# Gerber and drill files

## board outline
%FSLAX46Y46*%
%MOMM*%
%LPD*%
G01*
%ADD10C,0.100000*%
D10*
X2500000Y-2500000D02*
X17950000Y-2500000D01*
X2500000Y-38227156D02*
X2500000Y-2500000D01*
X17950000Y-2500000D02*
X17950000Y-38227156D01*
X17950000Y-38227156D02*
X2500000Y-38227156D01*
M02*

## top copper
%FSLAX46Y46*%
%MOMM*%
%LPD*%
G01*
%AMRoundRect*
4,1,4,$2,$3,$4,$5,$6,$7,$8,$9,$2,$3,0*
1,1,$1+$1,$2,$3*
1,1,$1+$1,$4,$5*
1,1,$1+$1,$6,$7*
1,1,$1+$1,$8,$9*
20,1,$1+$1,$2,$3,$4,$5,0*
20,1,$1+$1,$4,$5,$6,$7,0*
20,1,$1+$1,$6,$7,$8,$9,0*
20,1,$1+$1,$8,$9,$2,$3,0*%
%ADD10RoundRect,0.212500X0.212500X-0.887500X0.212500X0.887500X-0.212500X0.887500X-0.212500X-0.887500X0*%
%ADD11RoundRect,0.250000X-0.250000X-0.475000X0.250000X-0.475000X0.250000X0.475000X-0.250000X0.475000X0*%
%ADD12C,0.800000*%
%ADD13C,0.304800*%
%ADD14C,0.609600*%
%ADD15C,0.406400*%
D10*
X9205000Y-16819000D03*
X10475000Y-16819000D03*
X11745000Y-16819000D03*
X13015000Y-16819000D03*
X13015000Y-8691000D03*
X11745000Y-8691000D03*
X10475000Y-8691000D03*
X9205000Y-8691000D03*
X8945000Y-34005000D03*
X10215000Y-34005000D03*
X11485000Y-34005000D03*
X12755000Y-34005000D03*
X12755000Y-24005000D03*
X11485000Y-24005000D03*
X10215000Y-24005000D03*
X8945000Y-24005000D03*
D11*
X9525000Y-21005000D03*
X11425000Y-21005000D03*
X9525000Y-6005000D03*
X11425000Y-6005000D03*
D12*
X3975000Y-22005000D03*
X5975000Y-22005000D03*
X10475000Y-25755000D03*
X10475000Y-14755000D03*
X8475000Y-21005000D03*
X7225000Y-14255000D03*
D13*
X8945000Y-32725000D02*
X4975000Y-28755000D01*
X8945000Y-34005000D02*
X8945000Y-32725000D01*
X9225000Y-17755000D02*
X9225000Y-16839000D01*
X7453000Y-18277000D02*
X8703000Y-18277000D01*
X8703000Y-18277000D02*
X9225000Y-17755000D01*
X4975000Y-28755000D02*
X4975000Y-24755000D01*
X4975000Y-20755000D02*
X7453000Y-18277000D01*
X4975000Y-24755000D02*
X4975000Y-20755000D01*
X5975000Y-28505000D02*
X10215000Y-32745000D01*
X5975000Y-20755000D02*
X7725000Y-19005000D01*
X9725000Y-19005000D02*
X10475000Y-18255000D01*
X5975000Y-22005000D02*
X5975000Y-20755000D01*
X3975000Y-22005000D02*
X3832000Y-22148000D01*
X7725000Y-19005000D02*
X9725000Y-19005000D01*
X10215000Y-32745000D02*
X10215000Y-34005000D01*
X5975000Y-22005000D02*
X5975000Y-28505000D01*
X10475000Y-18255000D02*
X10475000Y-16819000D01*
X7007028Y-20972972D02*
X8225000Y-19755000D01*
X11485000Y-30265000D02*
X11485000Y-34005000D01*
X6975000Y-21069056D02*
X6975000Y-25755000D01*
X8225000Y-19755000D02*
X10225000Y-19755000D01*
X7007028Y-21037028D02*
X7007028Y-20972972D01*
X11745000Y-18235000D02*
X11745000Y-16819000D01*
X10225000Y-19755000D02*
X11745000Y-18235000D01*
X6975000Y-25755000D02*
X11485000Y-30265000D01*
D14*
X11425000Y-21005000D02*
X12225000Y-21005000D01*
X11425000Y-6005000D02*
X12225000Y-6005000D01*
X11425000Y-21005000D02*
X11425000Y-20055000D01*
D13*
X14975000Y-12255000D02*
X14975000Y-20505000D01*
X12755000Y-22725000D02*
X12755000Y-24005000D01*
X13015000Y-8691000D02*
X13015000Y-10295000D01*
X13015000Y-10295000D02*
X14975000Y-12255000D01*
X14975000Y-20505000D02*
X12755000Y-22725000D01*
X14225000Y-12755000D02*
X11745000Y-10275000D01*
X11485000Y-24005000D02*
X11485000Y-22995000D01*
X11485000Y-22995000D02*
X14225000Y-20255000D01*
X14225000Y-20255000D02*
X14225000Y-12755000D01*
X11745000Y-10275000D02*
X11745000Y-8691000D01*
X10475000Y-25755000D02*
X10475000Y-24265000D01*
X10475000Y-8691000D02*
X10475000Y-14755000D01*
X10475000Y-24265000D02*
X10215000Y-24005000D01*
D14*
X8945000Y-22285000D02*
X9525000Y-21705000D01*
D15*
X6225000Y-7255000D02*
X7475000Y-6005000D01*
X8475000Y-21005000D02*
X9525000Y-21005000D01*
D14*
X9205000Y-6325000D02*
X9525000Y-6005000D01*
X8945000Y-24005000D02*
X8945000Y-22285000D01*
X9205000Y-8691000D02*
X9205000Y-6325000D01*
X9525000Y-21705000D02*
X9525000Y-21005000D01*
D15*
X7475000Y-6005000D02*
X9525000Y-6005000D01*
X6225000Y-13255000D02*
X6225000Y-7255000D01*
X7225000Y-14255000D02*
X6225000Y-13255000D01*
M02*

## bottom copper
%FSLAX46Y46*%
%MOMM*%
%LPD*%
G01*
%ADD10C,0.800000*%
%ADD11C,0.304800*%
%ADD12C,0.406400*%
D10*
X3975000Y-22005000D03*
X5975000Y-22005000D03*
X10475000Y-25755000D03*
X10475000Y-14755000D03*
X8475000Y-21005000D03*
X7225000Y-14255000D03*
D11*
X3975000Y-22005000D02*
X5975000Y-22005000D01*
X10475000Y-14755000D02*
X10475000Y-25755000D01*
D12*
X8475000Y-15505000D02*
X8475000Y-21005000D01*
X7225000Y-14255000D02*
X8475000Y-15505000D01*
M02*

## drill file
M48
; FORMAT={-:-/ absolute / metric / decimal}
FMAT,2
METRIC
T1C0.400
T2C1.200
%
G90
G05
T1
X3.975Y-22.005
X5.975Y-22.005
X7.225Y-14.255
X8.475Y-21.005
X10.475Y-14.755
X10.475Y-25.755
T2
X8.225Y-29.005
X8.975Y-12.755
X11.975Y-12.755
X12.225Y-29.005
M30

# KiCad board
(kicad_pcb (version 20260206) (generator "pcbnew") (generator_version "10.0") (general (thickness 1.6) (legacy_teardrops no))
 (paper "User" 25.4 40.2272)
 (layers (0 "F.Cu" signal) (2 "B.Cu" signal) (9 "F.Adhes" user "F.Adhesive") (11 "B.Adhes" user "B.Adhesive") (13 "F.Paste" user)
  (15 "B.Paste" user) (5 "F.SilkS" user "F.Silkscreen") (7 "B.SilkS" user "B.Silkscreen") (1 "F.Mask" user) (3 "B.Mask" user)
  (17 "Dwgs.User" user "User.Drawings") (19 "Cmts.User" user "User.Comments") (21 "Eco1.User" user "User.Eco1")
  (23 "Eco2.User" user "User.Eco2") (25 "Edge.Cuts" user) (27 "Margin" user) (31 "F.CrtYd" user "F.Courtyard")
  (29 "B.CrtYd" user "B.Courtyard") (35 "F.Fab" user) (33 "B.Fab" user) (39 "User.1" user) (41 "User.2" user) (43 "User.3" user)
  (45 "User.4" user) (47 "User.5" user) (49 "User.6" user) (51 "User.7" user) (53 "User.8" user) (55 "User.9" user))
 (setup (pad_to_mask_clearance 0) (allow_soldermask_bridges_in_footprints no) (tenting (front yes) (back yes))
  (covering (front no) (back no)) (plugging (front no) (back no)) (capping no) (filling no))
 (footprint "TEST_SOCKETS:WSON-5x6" (layer "F.Cu") (at 10.475 12.755 90)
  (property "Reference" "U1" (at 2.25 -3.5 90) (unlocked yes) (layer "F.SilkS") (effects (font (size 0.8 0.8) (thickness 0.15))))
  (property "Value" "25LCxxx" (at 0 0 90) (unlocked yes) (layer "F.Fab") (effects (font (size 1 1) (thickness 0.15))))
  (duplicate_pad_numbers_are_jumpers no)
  (pad "" np_thru_hole circle (at 0 -1.5 90) (size 1.2 1.2) (drill 1.2) (layers "*.Cu" "*.Mask"))
  (pad "" np_thru_hole circle (at 0 1.5 90) (size 1.2 1.2) (drill 1.2) (layers "*.Cu" "*.Mask"))
  (pad "1" smd roundrect (at -4.064 -1.27 90) (size 2.2 0.85) (layers "F.Cu" "F.Mask" "F.Paste") (roundrect_rratio 0.25) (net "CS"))
  (pad "2" smd roundrect (at -4.064 0 90) (size 2.2 0.85) (layers "F.Cu" "F.Mask" "F.Paste") (roundrect_rratio 0.25) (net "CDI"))
  (pad "3" smd roundrect (at -4.064 1.27 90) (size 2.2 0.85) (layers "F.Cu" "F.Mask" "F.Paste") (roundrect_rratio 0.25) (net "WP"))
  (pad "4" smd roundrect (at -4.064 2.54 90) (size 2.2 0.85) (layers "F.Cu" "F.Mask" "F.Paste") (roundrect_rratio 0.25) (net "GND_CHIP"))
  (pad "5" smd roundrect (at 4.064 2.54 90) (size 2.2 0.85) (layers "F.Cu" "F.Mask" "F.Paste") (roundrect_rratio 0.25) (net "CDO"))
  (pad "6" smd roundrect (at 4.064 1.27 90) (size 2.2 0.85) (layers "F.Cu" "F.Mask" "F.Paste") (roundrect_rratio 0.25) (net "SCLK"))
  (pad "7" smd roundrect (at 4.064 0 90) (size 2.2 0.85) (layers "F.Cu" "F.Mask" "F.Paste") (roundrect_rratio 0.25) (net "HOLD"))
  (pad "8" smd roundrect (at 4.064 -1.27 90) (size 2.2 0.85) (layers "F.Cu" "F.Mask" "F.Paste") (roundrect_rratio 0.25) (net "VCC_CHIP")))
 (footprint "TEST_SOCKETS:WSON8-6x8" (layer "F.Cu") (at 10.225 29.005 90)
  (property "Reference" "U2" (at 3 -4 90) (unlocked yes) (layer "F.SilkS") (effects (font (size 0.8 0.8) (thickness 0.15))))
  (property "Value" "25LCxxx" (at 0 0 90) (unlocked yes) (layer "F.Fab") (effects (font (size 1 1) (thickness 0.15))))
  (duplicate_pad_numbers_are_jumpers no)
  (pad "" np_thru_hole circle (at 0 -2 90) (size 1.2 1.2) (drill 1.2) (layers "*.Cu" "*.Mask"))
  (pad "" np_thru_hole circle (at 0 2 90) (size 1.2 1.2) (drill 1.2) (layers "*.Cu" "*.Mask"))
  (pad "1" smd roundrect (at -5 -1.28 90) (size 2.2 0.85) (layers "F.Cu" "F.Mask" "F.Paste") (roundrect_rratio 0.25) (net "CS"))
  (pad "2" smd roundrect (at -5 -0.01 90) (size 2.2 0.85) (layers "F.Cu" "F.Mask" "F.Paste") (roundrect_rratio 0.25) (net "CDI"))
  (pad "3" smd roundrect (at -5 1.26 90) (size 2.2 0.85) (layers "F.Cu" "F.Mask" "F.Paste") (roundrect_rratio 0.25) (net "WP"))
  (pad "4" smd roundrect (at -5 2.53 90) (size 2.2 0.85) (layers "F.Cu" "F.Mask" "F.Paste") (roundrect_rratio 0.25) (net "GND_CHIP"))
  (pad "5" smd roundrect (at 5 2.53 90) (size 2.2 0.85) (layers "F.Cu" "F.Mask" "F.Paste") (roundrect_rratio 0.25) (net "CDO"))
  (pad "6" smd roundrect (at 5 1.26 90) (size 2.2 0.85) (layers "F.Cu" "F.Mask" "F.Paste") (roundrect_rratio 0.25) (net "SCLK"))
  (pad "7" smd roundrect (at 5 -0.01 90) (size 2.2 0.85) (layers "F.Cu" "F.Mask" "F.Paste") (roundrect_rratio 0.25) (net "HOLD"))
  (pad "8" smd roundrect (at 5 -1.28 90) (size 2.2 0.85) (layers "F.Cu" "F.Mask" "F.Paste") (roundrect_rratio 0.25) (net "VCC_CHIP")))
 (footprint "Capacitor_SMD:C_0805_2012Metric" (layer "F.Cu") (at 10.475 21.005)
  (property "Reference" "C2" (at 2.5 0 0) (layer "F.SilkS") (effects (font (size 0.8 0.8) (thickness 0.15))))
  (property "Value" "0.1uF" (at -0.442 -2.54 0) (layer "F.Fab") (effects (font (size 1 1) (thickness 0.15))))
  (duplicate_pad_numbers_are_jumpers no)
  (pad "1" smd roundrect (at -0.95 0) (size 1 1.45) (layers "F.Cu" "F.Mask" "F.Paste") (roundrect_rratio 0.25) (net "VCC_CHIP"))
  (pad "2" smd roundrect (at 0.95 0) (size 1 1.45) (layers "F.Cu" "F.Mask" "F.Paste") (roundrect_rratio 0.25) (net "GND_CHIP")))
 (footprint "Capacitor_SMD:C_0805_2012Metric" (layer "F.Cu") (at 10.475 6.005)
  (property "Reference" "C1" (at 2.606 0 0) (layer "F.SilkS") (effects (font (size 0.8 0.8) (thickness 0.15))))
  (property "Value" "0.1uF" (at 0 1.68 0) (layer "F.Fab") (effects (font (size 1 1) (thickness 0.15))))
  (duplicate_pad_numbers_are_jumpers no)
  (pad "1" smd roundrect (at -0.95 0) (size 1 1.45) (layers "F.Cu" "F.Mask" "F.Paste") (roundrect_rratio 0.25) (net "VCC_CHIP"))
  (pad "2" smd roundrect (at 0.95 0) (size 1 1.45) (layers "F.Cu" "F.Mask" "F.Paste") (roundrect_rratio 0.25) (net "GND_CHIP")))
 (gr_line (start 2.5 2.5) (end 17.95 2.5) (stroke (width 0.1) (type default)) (layer "Edge.Cuts"))
 (gr_line (start 2.5 38.227156) (end 2.5 2.5) (stroke (width 0.1) (type default)) (layer "Edge.Cuts"))
 (gr_line (start 17.95 2.5) (end 17.95 38.227156) (stroke (width 0.1) (type default)) (layer "Edge.Cuts"))
 (gr_line (start 17.95 38.227156) (end 2.5 38.227156) (stroke (width 0.1) (type default)) (layer "Edge.Cuts"))
 (segment (start 8.945 32.725) (end 4.975 28.755) (width 0.3048) (layer "F.Cu") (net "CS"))
 (segment (start 8.945 34.005) (end 8.945 32.725) (width 0.3048) (layer "F.Cu") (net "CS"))
 (segment (start 9.225 17.755) (end 9.225 16.839) (width 0.3048) (layer "F.Cu") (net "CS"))
 (segment (start 7.453 18.277) (end 8.703 18.277) (width 0.3048) (layer "F.Cu") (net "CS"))
 (segment (start 8.703 18.277) (end 9.225 17.755) (width 0.3048) (layer "F.Cu") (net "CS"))
 (segment (start 4.975 28.755) (end 4.975 24.755) (width 0.3048) (layer "F.Cu") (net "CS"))
 (segment (start 4.975 20.755) (end 7.453 18.277) (width 0.3048) (layer "F.Cu") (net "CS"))
 (segment (start 4.975 24.755) (end 4.975 20.755) (width 0.3048) (layer "F.Cu") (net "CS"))
 (segment (start 5.975 28.505) (end 10.215 32.745) (width 0.3048) (layer "F.Cu") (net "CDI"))
 (segment (start 5.975 20.755) (end 7.725 19.005) (width 0.3048) (layer "F.Cu") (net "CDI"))
 (segment (start 9.725 19.005) (end 10.475 18.255) (width 0.3048) (layer "F.Cu") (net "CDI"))
 (segment (start 5.975 22.005) (end 5.975 20.755) (width 0.3048) (layer "F.Cu") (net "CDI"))
 (segment (start 3.975 22.005) (end 3.832 22.148) (width 0.3048) (layer "F.Cu") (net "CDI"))
 (segment (start 7.725 19.005) (end 9.725 19.005) (width 0.3048) (layer "F.Cu") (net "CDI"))
 (segment (start 10.215 32.745) (end 10.215 34.005) (width 0.3048) (layer "F.Cu") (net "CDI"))
 (segment (start 5.975 22.005) (end 5.975 28.505) (width 0.3048) (layer "F.Cu") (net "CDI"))
 (segment (start 10.475 18.255) (end 10.475 16.819) (width 0.3048) (layer "F.Cu") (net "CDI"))
 (via (at 3.975 22.005) (size 0.8) (drill 0.4) (layers "F.Cu" "B.Cu") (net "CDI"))
 (via (at 5.975 22.005) (size 0.8) (drill 0.4) (layers "F.Cu" "B.Cu") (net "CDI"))
 (segment (start 3.975 22.005) (end 5.975 22.005) (width 0.3048) (layer "B.Cu") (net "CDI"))
 (segment (start 7.007028 20.972972) (end 8.225 19.755) (width 0.3048) (layer "F.Cu") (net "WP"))
 (segment (start 11.485 30.265) (end 11.485 34.005) (width 0.3048) (layer "F.Cu") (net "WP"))
 (segment (start 6.975 21.069056) (end 6.975 25.755) (width 0.3048) (layer "F.Cu") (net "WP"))
 (segment (start 8.225 19.755) (end 10.225 19.755) (width 0.3048) (layer "F.Cu") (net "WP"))
 (segment (start 7.007028 21.037028) (end 7.007028 20.972972) (width 0.3048) (layer "F.Cu") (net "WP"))
 (segment (start 11.745 18.235) (end 11.745 16.819) (width 0.3048) (layer "F.Cu") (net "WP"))
 (segment (start 10.225 19.755) (end 11.745 18.235) (width 0.3048) (layer "F.Cu") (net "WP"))
 (segment (start 6.975 25.755) (end 11.485 30.265) (width 0.3048) (layer "F.Cu") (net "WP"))
 (segment (start 11.425 21.005) (end 12.225 21.005) (width 0.6096) (layer "F.Cu") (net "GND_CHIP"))
 (segment (start 11.425 6.005) (end 12.225 6.005) (width 0.6096) (layer "F.Cu") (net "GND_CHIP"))
 (segment (start 11.425 21.005) (end 11.425 20.055) (width 0.6096) (layer "F.Cu") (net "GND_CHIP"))
 (segment (start 14.975 12.255) (end 14.975 20.505) (width 0.3048) (layer "F.Cu") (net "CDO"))
 (segment (start 12.755 22.725) (end 12.755 24.005) (width 0.3048) (layer "F.Cu") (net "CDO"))
 (segment (start 13.015 8.691) (end 13.015 10.295) (width 0.3048) (layer "F.Cu") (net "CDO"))
 (segment (start 13.015 10.295) (end 14.975 12.255) (width 0.3048) (layer "F.Cu") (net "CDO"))
 (segment (start 14.975 20.505) (end 12.755 22.725) (width 0.3048) (layer "F.Cu") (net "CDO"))
 (segment (start 14.225 12.755) (end 11.745 10.275) (width 0.3048) (layer "F.Cu") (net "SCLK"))
 (segment (start 11.485 24.005) (end 11.485 22.995) (width 0.3048) (layer "F.Cu") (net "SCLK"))
 (segment (start 11.485 22.995) (end 14.225 20.255) (width 0.3048) (layer "F.Cu") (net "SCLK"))
 (segment (start 14.225 20.255) (end 14.225 12.755) (width 0.3048) (layer "F.Cu") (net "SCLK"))
 (segment (start 11.745 10.275) (end 11.745 8.691) (width 0.3048) (layer "F.Cu") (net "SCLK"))
 (segment (start 10.475 25.755) (end 10.475 24.265) (width 0.3048) (layer "F.Cu") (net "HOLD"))
 (segment (start 10.475 8.691) (end 10.475 14.755) (width 0.3048) (layer "F.Cu") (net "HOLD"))
 (segment (start 10.475 24.265) (end 10.215 24.005) (width 0.3048) (layer "F.Cu") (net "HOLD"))
 (via (at 10.475 25.755) (size 0.8) (drill 0.4) (layers "F.Cu" "B.Cu") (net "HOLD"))
 (via (at 10.475 14.755) (size 0.8) (drill 0.4) (layers "F.Cu" "B.Cu") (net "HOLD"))
 (segment (start 10.475 14.755) (end 10.475 25.755) (width 0.3048) (layer "B.Cu") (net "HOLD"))
 (segment (start 8.945 22.285) (end 9.525 21.705) (width 0.6096) (layer "F.Cu") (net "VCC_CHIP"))
 (segment (start 6.225 7.255) (end 7.475 6.005) (width 0.4064) (layer "F.Cu") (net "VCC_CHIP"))
 (segment (start 8.475 21.005) (end 9.525 21.005) (width 0.4064) (layer "F.Cu") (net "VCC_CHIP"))
 (segment (start 9.205 6.325) (end 9.525 6.005) (width 0.6096) (layer "F.Cu") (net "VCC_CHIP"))
 (segment (start 8.945 24.005) (end 8.945 22.285) (width 0.6096) (layer "F.Cu") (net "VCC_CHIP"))
 (segment (start 9.205 8.691) (end 9.205 6.325) (width 0.6096) (layer "F.Cu") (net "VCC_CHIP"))
 (segment (start 9.525 21.705) (end 9.525 21.005) (width 0.6096) (layer "F.Cu") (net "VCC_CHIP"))
 (segment (start 7.475 6.005) (end 9.525 6.005) (width 0.4064) (layer "F.Cu") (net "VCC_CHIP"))
 (segment (start 6.225 13.255) (end 6.225 7.255) (width 0.4064) (layer "F.Cu") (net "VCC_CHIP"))
 (segment (start 7.225 14.255) (end 6.225 13.255) (width 0.4064) (layer "F.Cu") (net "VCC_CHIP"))
 (via (at 8.475 21.005) (size 0.8) (drill 0.4) (layers "F.Cu" "B.Cu") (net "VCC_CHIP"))
 (via (at 7.225 14.255) (size 0.8) (drill 0.4) (layers "F.Cu" "B.Cu") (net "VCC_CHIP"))
 (segment (start 8.475 15.505) (end 8.475 21.005) (width 0.4064) (layer "B.Cu") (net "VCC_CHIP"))
 (segment (start 7.225 14.255) (end 8.475 15.505) (width 0.4064) (layer "B.Cu") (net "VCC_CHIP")))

